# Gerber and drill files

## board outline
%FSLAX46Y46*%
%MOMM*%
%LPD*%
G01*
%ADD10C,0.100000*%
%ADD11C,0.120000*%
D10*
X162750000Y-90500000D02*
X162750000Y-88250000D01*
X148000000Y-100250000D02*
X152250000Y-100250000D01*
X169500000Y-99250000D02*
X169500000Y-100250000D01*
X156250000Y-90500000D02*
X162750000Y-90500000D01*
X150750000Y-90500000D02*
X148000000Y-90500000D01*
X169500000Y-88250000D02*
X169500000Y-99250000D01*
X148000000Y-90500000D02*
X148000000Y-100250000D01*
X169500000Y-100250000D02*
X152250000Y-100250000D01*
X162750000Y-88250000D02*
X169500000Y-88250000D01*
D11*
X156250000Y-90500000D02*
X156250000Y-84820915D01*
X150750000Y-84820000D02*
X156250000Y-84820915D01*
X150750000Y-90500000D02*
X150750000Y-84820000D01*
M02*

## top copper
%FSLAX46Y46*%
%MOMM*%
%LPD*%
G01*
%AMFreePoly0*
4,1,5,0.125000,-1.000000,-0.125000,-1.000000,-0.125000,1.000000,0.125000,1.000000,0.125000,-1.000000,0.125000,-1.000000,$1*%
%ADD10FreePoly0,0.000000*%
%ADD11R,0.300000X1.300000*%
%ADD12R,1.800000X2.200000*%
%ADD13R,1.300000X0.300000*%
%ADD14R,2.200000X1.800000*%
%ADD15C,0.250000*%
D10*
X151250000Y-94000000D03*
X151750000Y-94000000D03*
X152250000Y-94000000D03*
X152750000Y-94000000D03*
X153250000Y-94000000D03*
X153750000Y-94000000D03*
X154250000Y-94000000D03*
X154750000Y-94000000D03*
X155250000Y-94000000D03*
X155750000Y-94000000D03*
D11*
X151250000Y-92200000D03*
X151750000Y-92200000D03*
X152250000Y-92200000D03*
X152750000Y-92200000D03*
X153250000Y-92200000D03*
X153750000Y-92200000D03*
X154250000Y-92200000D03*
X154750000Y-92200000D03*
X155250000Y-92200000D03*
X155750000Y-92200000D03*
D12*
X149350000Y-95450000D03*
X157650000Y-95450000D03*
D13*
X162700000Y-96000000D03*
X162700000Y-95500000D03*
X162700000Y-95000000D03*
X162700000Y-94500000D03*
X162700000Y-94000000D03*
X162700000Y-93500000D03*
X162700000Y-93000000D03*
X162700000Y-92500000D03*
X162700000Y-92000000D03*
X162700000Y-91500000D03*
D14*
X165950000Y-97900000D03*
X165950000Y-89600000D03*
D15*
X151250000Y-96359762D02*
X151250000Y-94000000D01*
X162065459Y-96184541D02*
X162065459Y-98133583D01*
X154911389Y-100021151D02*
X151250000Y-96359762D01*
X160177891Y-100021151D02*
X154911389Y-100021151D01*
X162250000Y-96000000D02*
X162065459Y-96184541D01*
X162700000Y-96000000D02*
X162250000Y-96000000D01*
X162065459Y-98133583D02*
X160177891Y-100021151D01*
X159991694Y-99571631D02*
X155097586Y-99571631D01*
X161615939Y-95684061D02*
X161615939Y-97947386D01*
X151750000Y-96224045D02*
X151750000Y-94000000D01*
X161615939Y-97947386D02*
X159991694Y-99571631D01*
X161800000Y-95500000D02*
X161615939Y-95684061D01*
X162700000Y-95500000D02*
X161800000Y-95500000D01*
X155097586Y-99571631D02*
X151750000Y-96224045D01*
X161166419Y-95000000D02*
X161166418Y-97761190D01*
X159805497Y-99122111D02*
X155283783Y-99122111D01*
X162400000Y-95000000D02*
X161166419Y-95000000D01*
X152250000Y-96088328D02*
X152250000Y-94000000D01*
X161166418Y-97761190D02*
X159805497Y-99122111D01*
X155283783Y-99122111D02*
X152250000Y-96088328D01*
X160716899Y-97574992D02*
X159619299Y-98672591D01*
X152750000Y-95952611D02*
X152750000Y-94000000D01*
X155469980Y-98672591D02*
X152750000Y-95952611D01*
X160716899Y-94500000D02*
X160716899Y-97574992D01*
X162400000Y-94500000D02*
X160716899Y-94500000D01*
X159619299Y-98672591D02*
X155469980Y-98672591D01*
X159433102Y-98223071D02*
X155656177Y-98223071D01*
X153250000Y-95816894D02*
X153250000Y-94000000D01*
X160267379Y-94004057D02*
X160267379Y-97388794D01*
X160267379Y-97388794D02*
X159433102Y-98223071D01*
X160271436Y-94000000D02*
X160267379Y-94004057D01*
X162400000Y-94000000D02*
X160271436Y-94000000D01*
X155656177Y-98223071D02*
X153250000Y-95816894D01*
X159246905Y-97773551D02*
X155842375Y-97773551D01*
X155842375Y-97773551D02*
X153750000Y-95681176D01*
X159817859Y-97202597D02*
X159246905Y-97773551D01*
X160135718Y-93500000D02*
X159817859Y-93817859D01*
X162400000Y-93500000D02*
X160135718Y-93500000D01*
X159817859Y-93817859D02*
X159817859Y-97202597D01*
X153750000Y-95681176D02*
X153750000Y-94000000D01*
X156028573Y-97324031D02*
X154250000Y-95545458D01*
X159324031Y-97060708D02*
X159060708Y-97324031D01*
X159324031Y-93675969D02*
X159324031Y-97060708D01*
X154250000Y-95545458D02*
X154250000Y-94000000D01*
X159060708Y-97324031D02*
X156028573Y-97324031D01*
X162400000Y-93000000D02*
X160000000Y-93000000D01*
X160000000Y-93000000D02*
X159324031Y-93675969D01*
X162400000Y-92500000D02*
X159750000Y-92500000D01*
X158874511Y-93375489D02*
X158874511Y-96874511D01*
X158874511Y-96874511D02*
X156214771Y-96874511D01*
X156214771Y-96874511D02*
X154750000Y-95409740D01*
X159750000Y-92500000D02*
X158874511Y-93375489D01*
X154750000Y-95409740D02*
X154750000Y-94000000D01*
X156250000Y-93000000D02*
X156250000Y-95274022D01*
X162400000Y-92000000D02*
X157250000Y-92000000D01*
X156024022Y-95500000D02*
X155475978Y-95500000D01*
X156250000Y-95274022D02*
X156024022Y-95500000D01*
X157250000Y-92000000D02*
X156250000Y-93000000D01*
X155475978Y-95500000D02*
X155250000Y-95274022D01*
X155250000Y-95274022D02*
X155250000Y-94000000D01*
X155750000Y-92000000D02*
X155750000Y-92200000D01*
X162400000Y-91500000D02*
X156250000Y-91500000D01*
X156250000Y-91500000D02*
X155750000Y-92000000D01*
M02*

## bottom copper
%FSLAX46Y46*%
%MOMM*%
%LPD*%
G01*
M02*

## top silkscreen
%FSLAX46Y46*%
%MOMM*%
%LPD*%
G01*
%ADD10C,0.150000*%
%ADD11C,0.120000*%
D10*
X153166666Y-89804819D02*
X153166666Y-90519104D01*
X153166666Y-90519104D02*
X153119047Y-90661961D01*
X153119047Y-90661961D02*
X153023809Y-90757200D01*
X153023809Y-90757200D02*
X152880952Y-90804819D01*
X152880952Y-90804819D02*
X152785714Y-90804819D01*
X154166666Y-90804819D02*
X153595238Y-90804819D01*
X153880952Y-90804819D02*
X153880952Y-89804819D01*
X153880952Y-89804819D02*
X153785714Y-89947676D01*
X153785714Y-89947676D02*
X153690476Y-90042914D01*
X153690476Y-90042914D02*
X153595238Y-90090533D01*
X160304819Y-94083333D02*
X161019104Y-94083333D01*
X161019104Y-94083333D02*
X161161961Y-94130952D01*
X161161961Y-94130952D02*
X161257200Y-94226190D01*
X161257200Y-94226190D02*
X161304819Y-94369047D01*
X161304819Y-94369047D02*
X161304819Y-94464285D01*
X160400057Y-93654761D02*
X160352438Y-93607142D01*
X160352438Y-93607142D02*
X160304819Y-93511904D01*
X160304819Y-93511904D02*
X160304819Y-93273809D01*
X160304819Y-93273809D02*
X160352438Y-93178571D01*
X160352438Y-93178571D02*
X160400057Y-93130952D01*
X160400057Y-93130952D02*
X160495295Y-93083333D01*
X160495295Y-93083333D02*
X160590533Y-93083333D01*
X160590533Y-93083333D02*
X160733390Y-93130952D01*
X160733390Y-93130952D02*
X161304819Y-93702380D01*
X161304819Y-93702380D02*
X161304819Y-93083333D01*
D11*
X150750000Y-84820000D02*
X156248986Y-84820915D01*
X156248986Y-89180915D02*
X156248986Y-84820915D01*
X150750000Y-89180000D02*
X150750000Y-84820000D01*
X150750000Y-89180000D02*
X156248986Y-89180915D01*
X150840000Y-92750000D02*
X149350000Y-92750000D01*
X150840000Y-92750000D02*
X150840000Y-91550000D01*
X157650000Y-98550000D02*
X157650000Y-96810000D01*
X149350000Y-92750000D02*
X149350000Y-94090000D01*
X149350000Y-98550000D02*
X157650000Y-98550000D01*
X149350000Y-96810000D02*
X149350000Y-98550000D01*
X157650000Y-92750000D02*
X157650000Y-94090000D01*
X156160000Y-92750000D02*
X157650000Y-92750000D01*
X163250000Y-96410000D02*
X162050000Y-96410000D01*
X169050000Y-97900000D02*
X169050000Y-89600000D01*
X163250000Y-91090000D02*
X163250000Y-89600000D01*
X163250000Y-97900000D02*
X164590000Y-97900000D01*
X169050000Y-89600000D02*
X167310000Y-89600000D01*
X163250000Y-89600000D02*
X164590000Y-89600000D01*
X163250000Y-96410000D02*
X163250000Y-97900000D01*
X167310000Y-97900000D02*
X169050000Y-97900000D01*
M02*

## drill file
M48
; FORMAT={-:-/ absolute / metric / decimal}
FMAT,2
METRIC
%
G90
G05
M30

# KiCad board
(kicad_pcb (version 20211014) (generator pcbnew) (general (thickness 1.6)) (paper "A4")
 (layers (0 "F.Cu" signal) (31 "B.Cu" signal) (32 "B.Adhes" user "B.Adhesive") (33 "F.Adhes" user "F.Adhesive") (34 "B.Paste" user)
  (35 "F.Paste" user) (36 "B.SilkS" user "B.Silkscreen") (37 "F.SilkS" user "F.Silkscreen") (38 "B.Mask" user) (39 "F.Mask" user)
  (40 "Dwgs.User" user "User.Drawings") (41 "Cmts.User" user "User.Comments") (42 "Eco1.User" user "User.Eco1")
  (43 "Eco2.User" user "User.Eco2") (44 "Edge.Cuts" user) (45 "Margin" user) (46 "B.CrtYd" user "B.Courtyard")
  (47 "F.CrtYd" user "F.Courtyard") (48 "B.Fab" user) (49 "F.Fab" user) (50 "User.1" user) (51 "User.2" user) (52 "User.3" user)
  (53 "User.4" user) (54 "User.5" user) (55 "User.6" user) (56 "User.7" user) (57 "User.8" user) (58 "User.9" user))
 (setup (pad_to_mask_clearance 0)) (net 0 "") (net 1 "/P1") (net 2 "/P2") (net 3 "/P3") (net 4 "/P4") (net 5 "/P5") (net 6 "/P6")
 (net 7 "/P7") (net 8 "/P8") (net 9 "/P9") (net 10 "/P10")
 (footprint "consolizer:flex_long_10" (layer "F.Cu") (at 153.75 89)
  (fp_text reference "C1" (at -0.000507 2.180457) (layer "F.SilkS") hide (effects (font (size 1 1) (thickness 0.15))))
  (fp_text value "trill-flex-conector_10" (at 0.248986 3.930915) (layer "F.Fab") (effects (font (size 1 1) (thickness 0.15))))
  (fp_line (start -3 -4.18) (end 2.498986 -4.179085) (layer "F.SilkS") (width 0.12))
  (fp_line (start 2.498986 0.180915) (end 2.498986 -4.179085) (layer "F.SilkS") (width 0.12))
  (fp_line (start -3 0.18) (end -3 -4.18) (layer "F.SilkS") (width 0.12))
  (fp_line (start -3 0.18) (end 2.498986 0.180915) (layer "F.SilkS") (width 0.12))
  (fp_line (start 2.5 1.5) (end 2.5 -4.179085) (layer "Edge.Cuts") (width 0.12))
  (fp_line (start -3 -4.18) (end 2.5 -4.179085) (layer "Edge.Cuts") (width 0.12))
  (fp_line (start -3 1.5) (end -3 -4.18) (layer "Edge.Cuts") (width 0.12))
  (pad "" smd rect (at -2 -2) (size 0.25 4) (layers "F.Paste" "F.Mask"))
  (pad "" smd rect (at 1.5 -2) (size 0.25 4) (layers "F.Paste" "F.Mask"))
  (pad "" smd rect (at 0.5 -2) (size 0.25 4) (layers "F.Paste" "F.Mask"))
  (pad "" smd rect (at 1 -2) (size 0.25 4) (layers "F.Paste" "F.Mask"))
  (pad "" smd rect (at -0.5 -2) (size 0.25 4) (layers "F.Paste" "F.Mask"))
  (pad "" smd rect (at 0 -2) (size 0.25 4) (layers "F.Paste" "F.Mask"))
  (pad "" smd rect (at -1.5 -2) (size 0.25 4) (layers "F.Paste" "F.Mask"))
  (pad "" smd rect (at -1 -2) (size 0.25 4) (layers "F.Paste" "F.Mask"))
  (pad "" smd rect (at 1.998986 -1.999085) (size 0.25 4) (layers "F.Paste" "F.Mask"))
  (pad "" smd rect (at -2.5 -2) (size 0.25 4) (layers "F.Paste" "F.Mask"))
  (pad "1" smd custom (at -2.5 5) (size 0.25 2) (layers "F.Cu") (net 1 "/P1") (zone_connect 0) (options (clearance outline) (anchor rect))
   (primitives))
  (pad "2" smd custom (at -2 5) (size 0.25 2) (layers "F.Cu") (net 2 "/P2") (zone_connect 0) (options (clearance outline) (anchor rect))
   (primitives))
  (pad "3" smd custom (at -1.5 5) (size 0.25 2) (layers "F.Cu") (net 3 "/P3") (zone_connect 0) (options (clearance outline) (anchor rect))
   (primitives))
  (pad "4" smd custom (at -1 5) (size 0.25 2) (layers "F.Cu") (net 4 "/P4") (zone_connect 0) (options (clearance outline) (anchor rect))
   (primitives))
  (pad "5" smd custom (at -0.5 5) (size 0.25 2) (layers "F.Cu") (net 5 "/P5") (zone_connect 0) (options (clearance outline) (anchor rect))
   (primitives))
  (pad "6" smd custom (at 0 5) (size 0.25 2) (layers "F.Cu") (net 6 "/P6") (zone_connect 0) (options (clearance outline) (anchor rect))
   (primitives))
  (pad "7" smd custom (at 0.5 5) (size 0.25 2) (layers "F.Cu") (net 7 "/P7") (zone_connect 0) (options (clearance outline) (anchor rect))
   (primitives))
  (pad "8" smd custom (at 1 5) (size 0.25 2) (layers "F.Cu") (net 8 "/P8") (zone_connect 0) (options (clearance outline) (anchor rect))
   (primitives))
  (pad "9" smd custom (at 1.5 5) (size 0.25 2) (layers "F.Cu") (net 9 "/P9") (zone_connect 0) (options (clearance outline) (anchor rect))
   (primitives))
  (pad "10" smd custom (at 2 5) (size 0.25 2) (layers "F.Cu") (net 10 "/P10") (zone_connect 0) (options (clearance outline) (anchor rect))
   (primitives)))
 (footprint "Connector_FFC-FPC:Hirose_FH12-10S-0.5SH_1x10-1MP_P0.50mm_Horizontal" (layer "F.Cu") (at 153.5 94.05)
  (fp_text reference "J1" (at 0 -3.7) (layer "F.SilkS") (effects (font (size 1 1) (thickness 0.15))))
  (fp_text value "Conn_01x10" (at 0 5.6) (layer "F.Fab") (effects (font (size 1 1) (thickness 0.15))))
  (fp_line (start -2.66 -1.3) (end -4.15 -1.3) (layer "F.SilkS") (width 0.12))
  (fp_line (start -2.66 -1.3) (end -2.66 -2.5) (layer "F.SilkS") (width 0.12))
  (fp_line (start 4.15 4.5) (end 4.15 2.76) (layer "F.SilkS") (width 0.12))
  (fp_line (start -4.15 -1.3) (end -4.15 0.04) (layer "F.SilkS") (width 0.12))
  (fp_line (start -4.15 4.5) (end 4.15 4.5) (layer "F.SilkS") (width 0.12))
  (fp_line (start -4.15 2.76) (end -4.15 4.5) (layer "F.SilkS") (width 0.12))
  (fp_line (start 4.15 -1.3) (end 4.15 0.04) (layer "F.SilkS") (width 0.12))
  (fp_line (start 2.66 -1.3) (end 4.15 -1.3) (layer "F.SilkS") (width 0.12))
  (pad "1" smd rect (at -2.25 -1.85) (size 0.3 1.3) (layers "F.Cu" "F.Paste" "F.Mask") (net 1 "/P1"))
  (pad "2" smd rect (at -1.75 -1.85) (size 0.3 1.3) (layers "F.Cu" "F.Paste" "F.Mask") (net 2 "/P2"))
  (pad "3" smd rect (at -1.25 -1.85) (size 0.3 1.3) (layers "F.Cu" "F.Paste" "F.Mask") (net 3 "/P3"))
  (pad "4" smd rect (at -0.75 -1.85) (size 0.3 1.3) (layers "F.Cu" "F.Paste" "F.Mask") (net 4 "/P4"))
  (pad "5" smd rect (at -0.25 -1.85) (size 0.3 1.3) (layers "F.Cu" "F.Paste" "F.Mask") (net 5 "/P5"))
  (pad "6" smd rect (at 0.25 -1.85) (size 0.3 1.3) (layers "F.Cu" "F.Paste" "F.Mask") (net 6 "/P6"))
  (pad "7" smd rect (at 0.75 -1.85) (size 0.3 1.3) (layers "F.Cu" "F.Paste" "F.Mask") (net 7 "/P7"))
  (pad "8" smd rect (at 1.25 -1.85) (size 0.3 1.3) (layers "F.Cu" "F.Paste" "F.Mask") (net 8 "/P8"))
  (pad "9" smd rect (at 1.75 -1.85) (size 0.3 1.3) (layers "F.Cu" "F.Paste" "F.Mask") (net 9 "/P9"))
  (pad "10" smd rect (at 2.25 -1.85) (size 0.3 1.3) (layers "F.Cu" "F.Paste" "F.Mask") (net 10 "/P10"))
  (pad "MP" smd rect (at -4.15 1.4) (size 1.8 2.2) (layers "F.Cu" "F.Paste" "F.Mask"))
  (pad "MP" smd rect (at 4.15 1.4) (size 1.8 2.2) (layers "F.Cu" "F.Paste" "F.Mask")))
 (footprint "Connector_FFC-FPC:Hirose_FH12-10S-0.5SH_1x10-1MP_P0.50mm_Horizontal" (layer "F.Cu") (at 164.55 93.75 90)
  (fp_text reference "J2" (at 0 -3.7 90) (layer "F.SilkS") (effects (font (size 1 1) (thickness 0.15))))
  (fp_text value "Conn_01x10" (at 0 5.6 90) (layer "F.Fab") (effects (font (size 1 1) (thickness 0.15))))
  (fp_line (start -2.66 -1.3) (end -2.66 -2.5) (layer "F.SilkS") (width 0.12))
  (fp_line (start -4.15 4.5) (end 4.15 4.5) (layer "F.SilkS") (width 0.12))
  (fp_line (start 2.66 -1.3) (end 4.15 -1.3) (layer "F.SilkS") (width 0.12))
  (fp_line (start -4.15 -1.3) (end -4.15 0.04) (layer "F.SilkS") (width 0.12))
  (fp_line (start 4.15 4.5) (end 4.15 2.76) (layer "F.SilkS") (width 0.12))
  (fp_line (start 4.15 -1.3) (end 4.15 0.04) (layer "F.SilkS") (width 0.12))
  (fp_line (start -2.66 -1.3) (end -4.15 -1.3) (layer "F.SilkS") (width 0.12))
  (fp_line (start -4.15 2.76) (end -4.15 4.5) (layer "F.SilkS") (width 0.12))
  (pad "1" smd rect (at -2.25 -1.85 90) (size 0.3 1.3) (layers "F.Cu" "F.Paste" "F.Mask") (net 1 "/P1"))
  (pad "2" smd rect (at -1.75 -1.85 90) (size 0.3 1.3) (layers "F.Cu" "F.Paste" "F.Mask") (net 2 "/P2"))
  (pad "3" smd rect (at -1.25 -1.85 90) (size 0.3 1.3) (layers "F.Cu" "F.Paste" "F.Mask") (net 3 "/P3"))
  (pad "4" smd rect (at -0.75 -1.85 90) (size 0.3 1.3) (layers "F.Cu" "F.Paste" "F.Mask") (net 4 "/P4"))
  (pad "5" smd rect (at -0.25 -1.85 90) (size 0.3 1.3) (layers "F.Cu" "F.Paste" "F.Mask") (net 5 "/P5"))
  (pad "6" smd rect (at 0.25 -1.85 90) (size 0.3 1.3) (layers "F.Cu" "F.Paste" "F.Mask") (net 6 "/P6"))
  (pad "7" smd rect (at 0.75 -1.85 90) (size 0.3 1.3) (layers "F.Cu" "F.Paste" "F.Mask") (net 7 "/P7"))
  (pad "8" smd rect (at 1.25 -1.85 90) (size 0.3 1.3) (layers "F.Cu" "F.Paste" "F.Mask") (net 8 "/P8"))
  (pad "9" smd rect (at 1.75 -1.85 90) (size 0.3 1.3) (layers "F.Cu" "F.Paste" "F.Mask") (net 9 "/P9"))
  (pad "10" smd rect (at 2.25 -1.85 90) (size 0.3 1.3) (layers "F.Cu" "F.Paste" "F.Mask") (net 10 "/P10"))
  (pad "MP" smd rect (at -4.15 1.4 90) (size 1.8 2.2) (layers "F.Cu" "F.Paste" "F.Mask"))
  (pad "MP" smd rect (at 4.15 1.4 90) (size 1.8 2.2) (layers "F.Cu" "F.Paste" "F.Mask")))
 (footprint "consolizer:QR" (layer "B.Cu") (at 163 95.25 -90)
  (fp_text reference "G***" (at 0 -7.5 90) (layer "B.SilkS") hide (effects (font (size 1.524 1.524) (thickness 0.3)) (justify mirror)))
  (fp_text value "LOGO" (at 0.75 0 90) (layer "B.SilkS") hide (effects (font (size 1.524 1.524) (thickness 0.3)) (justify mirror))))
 (gr_line (start 162.75 90.5) (end 162.75 88.25) (layer "Edge.Cuts") (width 0.1))
 (gr_line (start 148 100.25) (end 152.25 100.25) (layer "Edge.Cuts") (width 0.1))
 (gr_line (start 169.5 99.25) (end 169.5 100.25) (layer "Edge.Cuts") (width 0.1))
 (gr_line (start 156.25 90.5) (end 162.75 90.5) (layer "Edge.Cuts") (width 0.1))
 (gr_line (start 150.75 90.5) (end 148 90.5) (layer "Edge.Cuts") (width 0.1))
 (gr_line (start 169.5 88.25) (end 169.5 99.25) (layer "Edge.Cuts") (width 0.1))
 (gr_line (start 148 90.5) (end 148 100.25) (layer "Edge.Cuts") (width 0.1))
 (gr_line (start 169.5 100.25) (end 152.25 100.25) (layer "Edge.Cuts") (width 0.1))
 (gr_line (start 162.75 88.25) (end 169.5 88.25) (layer "Edge.Cuts") (width 0.1))
 (segment (start 151.25 96.359762) (end 151.25 94) (width 0.25) (layer "F.Cu") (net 1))
 (segment (start 162.065459 96.184541) (end 162.065459 98.133583) (width 0.25) (layer "F.Cu") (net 1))
 (segment (start 154.911389 100.021151) (end 151.25 96.359762) (width 0.25) (layer "F.Cu") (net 1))
 (segment (start 160.177891 100.021151) (end 154.911389 100.021151) (width 0.25) (layer "F.Cu") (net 1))
 (segment (start 162.25 96) (end 162.065459 96.184541) (width 0.25) (layer "F.Cu") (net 1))
 (segment (start 162.7 96) (end 162.25 96) (width 0.25) (layer "F.Cu") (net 1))
 (segment (start 162.065459 98.133583) (end 160.177891 100.021151) (width 0.25) (layer "F.Cu") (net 1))
 (segment (start 159.991694 99.571631) (end 155.097586 99.571631) (width 0.25) (layer "F.Cu") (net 2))
 (segment (start 161.615939 95.684061) (end 161.615939 97.947386) (width 0.25) (layer "F.Cu") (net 2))
 (segment (start 151.75 96.224045) (end 151.75 94) (width 0.25) (layer "F.Cu") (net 2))
 (segment (start 161.615939 97.947386) (end 159.991694 99.571631) (width 0.25) (layer "F.Cu") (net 2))
 (segment (start 161.8 95.5) (end 161.615939 95.684061) (width 0.25) (layer "F.Cu") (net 2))
 (segment (start 162.7 95.5) (end 161.8 95.5) (width 0.25) (layer "F.Cu") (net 2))
 (segment (start 155.097586 99.571631) (end 151.75 96.224045) (width 0.25) (layer "F.Cu") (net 2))
 (segment (start 161.166419 95) (end 161.166418 97.76119) (width 0.25) (layer "F.Cu") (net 3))
 (segment (start 159.805497 99.122111) (end 155.283783 99.122111) (width 0.25) (layer "F.Cu") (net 3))
 (segment (start 162.4 95) (end 161.166419 95) (width 0.25) (layer "F.Cu") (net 3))
 (segment (start 152.25 96.088328) (end 152.25 94) (width 0.25) (layer "F.Cu") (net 3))
 (segment (start 161.166418 97.76119) (end 159.805497 99.122111) (width 0.25) (layer "F.Cu") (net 3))
 (segment (start 155.283783 99.122111) (end 152.25 96.088328) (width 0.25) (layer "F.Cu") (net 3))
 (segment (start 160.716899 97.574992) (end 159.619299 98.672591) (width 0.25) (layer "F.Cu") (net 4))
 (segment (start 152.75 95.952611) (end 152.75 94) (width 0.25) (layer "F.Cu") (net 4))
 (segment (start 155.46998 98.672591) (end 152.75 95.952611) (width 0.25) (layer "F.Cu") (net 4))
 (segment (start 160.716899 94.5) (end 160.716899 97.574992) (width 0.25) (layer "F.Cu") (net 4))
 (segment (start 162.4 94.5) (end 160.716899 94.5) (width 0.25) (layer "F.Cu") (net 4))
 (segment (start 159.619299 98.672591) (end 155.46998 98.672591) (width 0.25) (layer "F.Cu") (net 4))
 (segment (start 159.433102 98.223071) (end 155.656177 98.223071) (width 0.25) (layer "F.Cu") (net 5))
 (segment (start 153.25 95.816894) (end 153.25 94) (width 0.25) (layer "F.Cu") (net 5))
 (segment (start 160.267379 94.004057) (end 160.267379 97.388794) (width 0.25) (layer "F.Cu") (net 5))
 (segment (start 160.267379 97.388794) (end 159.433102 98.223071) (width 0.25) (layer "F.Cu") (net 5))
 (segment (start 160.271436 94) (end 160.267379 94.004057) (width 0.25) (layer "F.Cu") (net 5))
 (segment (start 162.4 94) (end 160.271436 94) (width 0.25) (layer "F.Cu") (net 5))
 (segment (start 155.656177 98.223071) (end 153.25 95.816894) (width 0.25) (layer "F.Cu") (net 5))
 (segment (start 159.246905 97.773551) (end 155.842375 97.773551) (width 0.25) (layer "F.Cu") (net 6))
 (segment (start 155.842375 97.773551) (end 153.75 95.681176) (width 0.25) (layer "F.Cu") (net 6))
 (segment (start 159.817859 97.202597) (end 159.246905 97.773551) (width 0.25) (layer "F.Cu") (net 6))
 (segment (start 160.135718 93.5) (end 159.817859 93.817859) (width 0.25) (layer "F.Cu") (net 6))
 (segment (start 162.4 93.5) (end 160.135718 93.5) (width 0.25) (layer "F.Cu") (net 6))
 (segment (start 159.817859 93.817859) (end 159.817859 97.202597) (width 0.25) (layer "F.Cu") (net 6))
 (segment (start 153.75 95.681176) (end 153.75 94) (width 0.25) (layer "F.Cu") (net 6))
 (segment (start 156.028573 97.324031) (end 154.25 95.545458) (width 0.25) (layer "F.Cu") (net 7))
 (segment (start 159.324031 97.060708) (end 159.060708 97.324031) (width 0.25) (layer "F.Cu") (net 7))
 (segment (start 159.324031 93.675969) (end 159.324031 97.060708) (width 0.25) (layer "F.Cu") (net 7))
 (segment (start 154.25 95.545458) (end 154.25 94) (width 0.25) (layer "F.Cu") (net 7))
 (segment (start 159.060708 97.324031) (end 156.028573 97.324031) (width 0.25) (layer "F.Cu") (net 7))
 (segment (start 162.4 93) (end 160 93) (width 0.25) (layer "F.Cu") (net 7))
 (segment (start 160 93) (end 159.324031 93.675969) (width 0.25) (layer "F.Cu") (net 7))
 (segment (start 162.4 92.5) (end 159.75 92.5) (width 0.25) (layer "F.Cu") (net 8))
 (segment (start 158.874511 93.375489) (end 158.874511 96.874511) (width 0.25) (layer "F.Cu") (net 8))
 (segment (start 158.874511 96.874511) (end 156.214771 96.874511) (width 0.25) (layer "F.Cu") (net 8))
 (segment (start 156.214771 96.874511) (end 154.75 95.40974) (width 0.25) (layer "F.Cu") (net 8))
 (segment (start 159.75 92.5) (end 158.874511 93.375489) (width 0.25) (layer "F.Cu") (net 8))
 (segment (start 154.75 95.40974) (end 154.75 94) (width 0.25) (layer "F.Cu") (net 8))
 (segment (start 156.25 93) (end 156.25 95.274022) (width 0.25) (layer "F.Cu") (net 9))
 (segment (start 162.4 92) (end 157.25 92) (width 0.25) (layer "F.Cu") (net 9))
 (segment (start 156.024022 95.5) (end 155.475978 95.5) (width 0.25) (layer "F.Cu") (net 9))
 (segment (start 156.25 95.274022) (end 156.024022 95.5) (width 0.25) (layer "F.Cu") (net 9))
 (segment (start 157.25 92) (end 156.25 93) (width 0.25) (layer "F.Cu") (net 9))
 (segment (start 155.475978 95.5) (end 155.25 95.274022) (width 0.25) (layer "F.Cu") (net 9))
 (segment (start 155.25 95.274022) (end 155.25 94) (width 0.25) (layer "F.Cu") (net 9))
 (segment (start 155.75 92) (end 155.75 92.2) (width 0.25) (layer "F.Cu") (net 10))
 (segment (start 162.4 91.5) (end 156.25 91.5) (width 0.25) (layer "F.Cu") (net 10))
 (segment (start 156.25 91.5) (end 155.75 92) (width 0.25) (layer "F.Cu") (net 10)))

